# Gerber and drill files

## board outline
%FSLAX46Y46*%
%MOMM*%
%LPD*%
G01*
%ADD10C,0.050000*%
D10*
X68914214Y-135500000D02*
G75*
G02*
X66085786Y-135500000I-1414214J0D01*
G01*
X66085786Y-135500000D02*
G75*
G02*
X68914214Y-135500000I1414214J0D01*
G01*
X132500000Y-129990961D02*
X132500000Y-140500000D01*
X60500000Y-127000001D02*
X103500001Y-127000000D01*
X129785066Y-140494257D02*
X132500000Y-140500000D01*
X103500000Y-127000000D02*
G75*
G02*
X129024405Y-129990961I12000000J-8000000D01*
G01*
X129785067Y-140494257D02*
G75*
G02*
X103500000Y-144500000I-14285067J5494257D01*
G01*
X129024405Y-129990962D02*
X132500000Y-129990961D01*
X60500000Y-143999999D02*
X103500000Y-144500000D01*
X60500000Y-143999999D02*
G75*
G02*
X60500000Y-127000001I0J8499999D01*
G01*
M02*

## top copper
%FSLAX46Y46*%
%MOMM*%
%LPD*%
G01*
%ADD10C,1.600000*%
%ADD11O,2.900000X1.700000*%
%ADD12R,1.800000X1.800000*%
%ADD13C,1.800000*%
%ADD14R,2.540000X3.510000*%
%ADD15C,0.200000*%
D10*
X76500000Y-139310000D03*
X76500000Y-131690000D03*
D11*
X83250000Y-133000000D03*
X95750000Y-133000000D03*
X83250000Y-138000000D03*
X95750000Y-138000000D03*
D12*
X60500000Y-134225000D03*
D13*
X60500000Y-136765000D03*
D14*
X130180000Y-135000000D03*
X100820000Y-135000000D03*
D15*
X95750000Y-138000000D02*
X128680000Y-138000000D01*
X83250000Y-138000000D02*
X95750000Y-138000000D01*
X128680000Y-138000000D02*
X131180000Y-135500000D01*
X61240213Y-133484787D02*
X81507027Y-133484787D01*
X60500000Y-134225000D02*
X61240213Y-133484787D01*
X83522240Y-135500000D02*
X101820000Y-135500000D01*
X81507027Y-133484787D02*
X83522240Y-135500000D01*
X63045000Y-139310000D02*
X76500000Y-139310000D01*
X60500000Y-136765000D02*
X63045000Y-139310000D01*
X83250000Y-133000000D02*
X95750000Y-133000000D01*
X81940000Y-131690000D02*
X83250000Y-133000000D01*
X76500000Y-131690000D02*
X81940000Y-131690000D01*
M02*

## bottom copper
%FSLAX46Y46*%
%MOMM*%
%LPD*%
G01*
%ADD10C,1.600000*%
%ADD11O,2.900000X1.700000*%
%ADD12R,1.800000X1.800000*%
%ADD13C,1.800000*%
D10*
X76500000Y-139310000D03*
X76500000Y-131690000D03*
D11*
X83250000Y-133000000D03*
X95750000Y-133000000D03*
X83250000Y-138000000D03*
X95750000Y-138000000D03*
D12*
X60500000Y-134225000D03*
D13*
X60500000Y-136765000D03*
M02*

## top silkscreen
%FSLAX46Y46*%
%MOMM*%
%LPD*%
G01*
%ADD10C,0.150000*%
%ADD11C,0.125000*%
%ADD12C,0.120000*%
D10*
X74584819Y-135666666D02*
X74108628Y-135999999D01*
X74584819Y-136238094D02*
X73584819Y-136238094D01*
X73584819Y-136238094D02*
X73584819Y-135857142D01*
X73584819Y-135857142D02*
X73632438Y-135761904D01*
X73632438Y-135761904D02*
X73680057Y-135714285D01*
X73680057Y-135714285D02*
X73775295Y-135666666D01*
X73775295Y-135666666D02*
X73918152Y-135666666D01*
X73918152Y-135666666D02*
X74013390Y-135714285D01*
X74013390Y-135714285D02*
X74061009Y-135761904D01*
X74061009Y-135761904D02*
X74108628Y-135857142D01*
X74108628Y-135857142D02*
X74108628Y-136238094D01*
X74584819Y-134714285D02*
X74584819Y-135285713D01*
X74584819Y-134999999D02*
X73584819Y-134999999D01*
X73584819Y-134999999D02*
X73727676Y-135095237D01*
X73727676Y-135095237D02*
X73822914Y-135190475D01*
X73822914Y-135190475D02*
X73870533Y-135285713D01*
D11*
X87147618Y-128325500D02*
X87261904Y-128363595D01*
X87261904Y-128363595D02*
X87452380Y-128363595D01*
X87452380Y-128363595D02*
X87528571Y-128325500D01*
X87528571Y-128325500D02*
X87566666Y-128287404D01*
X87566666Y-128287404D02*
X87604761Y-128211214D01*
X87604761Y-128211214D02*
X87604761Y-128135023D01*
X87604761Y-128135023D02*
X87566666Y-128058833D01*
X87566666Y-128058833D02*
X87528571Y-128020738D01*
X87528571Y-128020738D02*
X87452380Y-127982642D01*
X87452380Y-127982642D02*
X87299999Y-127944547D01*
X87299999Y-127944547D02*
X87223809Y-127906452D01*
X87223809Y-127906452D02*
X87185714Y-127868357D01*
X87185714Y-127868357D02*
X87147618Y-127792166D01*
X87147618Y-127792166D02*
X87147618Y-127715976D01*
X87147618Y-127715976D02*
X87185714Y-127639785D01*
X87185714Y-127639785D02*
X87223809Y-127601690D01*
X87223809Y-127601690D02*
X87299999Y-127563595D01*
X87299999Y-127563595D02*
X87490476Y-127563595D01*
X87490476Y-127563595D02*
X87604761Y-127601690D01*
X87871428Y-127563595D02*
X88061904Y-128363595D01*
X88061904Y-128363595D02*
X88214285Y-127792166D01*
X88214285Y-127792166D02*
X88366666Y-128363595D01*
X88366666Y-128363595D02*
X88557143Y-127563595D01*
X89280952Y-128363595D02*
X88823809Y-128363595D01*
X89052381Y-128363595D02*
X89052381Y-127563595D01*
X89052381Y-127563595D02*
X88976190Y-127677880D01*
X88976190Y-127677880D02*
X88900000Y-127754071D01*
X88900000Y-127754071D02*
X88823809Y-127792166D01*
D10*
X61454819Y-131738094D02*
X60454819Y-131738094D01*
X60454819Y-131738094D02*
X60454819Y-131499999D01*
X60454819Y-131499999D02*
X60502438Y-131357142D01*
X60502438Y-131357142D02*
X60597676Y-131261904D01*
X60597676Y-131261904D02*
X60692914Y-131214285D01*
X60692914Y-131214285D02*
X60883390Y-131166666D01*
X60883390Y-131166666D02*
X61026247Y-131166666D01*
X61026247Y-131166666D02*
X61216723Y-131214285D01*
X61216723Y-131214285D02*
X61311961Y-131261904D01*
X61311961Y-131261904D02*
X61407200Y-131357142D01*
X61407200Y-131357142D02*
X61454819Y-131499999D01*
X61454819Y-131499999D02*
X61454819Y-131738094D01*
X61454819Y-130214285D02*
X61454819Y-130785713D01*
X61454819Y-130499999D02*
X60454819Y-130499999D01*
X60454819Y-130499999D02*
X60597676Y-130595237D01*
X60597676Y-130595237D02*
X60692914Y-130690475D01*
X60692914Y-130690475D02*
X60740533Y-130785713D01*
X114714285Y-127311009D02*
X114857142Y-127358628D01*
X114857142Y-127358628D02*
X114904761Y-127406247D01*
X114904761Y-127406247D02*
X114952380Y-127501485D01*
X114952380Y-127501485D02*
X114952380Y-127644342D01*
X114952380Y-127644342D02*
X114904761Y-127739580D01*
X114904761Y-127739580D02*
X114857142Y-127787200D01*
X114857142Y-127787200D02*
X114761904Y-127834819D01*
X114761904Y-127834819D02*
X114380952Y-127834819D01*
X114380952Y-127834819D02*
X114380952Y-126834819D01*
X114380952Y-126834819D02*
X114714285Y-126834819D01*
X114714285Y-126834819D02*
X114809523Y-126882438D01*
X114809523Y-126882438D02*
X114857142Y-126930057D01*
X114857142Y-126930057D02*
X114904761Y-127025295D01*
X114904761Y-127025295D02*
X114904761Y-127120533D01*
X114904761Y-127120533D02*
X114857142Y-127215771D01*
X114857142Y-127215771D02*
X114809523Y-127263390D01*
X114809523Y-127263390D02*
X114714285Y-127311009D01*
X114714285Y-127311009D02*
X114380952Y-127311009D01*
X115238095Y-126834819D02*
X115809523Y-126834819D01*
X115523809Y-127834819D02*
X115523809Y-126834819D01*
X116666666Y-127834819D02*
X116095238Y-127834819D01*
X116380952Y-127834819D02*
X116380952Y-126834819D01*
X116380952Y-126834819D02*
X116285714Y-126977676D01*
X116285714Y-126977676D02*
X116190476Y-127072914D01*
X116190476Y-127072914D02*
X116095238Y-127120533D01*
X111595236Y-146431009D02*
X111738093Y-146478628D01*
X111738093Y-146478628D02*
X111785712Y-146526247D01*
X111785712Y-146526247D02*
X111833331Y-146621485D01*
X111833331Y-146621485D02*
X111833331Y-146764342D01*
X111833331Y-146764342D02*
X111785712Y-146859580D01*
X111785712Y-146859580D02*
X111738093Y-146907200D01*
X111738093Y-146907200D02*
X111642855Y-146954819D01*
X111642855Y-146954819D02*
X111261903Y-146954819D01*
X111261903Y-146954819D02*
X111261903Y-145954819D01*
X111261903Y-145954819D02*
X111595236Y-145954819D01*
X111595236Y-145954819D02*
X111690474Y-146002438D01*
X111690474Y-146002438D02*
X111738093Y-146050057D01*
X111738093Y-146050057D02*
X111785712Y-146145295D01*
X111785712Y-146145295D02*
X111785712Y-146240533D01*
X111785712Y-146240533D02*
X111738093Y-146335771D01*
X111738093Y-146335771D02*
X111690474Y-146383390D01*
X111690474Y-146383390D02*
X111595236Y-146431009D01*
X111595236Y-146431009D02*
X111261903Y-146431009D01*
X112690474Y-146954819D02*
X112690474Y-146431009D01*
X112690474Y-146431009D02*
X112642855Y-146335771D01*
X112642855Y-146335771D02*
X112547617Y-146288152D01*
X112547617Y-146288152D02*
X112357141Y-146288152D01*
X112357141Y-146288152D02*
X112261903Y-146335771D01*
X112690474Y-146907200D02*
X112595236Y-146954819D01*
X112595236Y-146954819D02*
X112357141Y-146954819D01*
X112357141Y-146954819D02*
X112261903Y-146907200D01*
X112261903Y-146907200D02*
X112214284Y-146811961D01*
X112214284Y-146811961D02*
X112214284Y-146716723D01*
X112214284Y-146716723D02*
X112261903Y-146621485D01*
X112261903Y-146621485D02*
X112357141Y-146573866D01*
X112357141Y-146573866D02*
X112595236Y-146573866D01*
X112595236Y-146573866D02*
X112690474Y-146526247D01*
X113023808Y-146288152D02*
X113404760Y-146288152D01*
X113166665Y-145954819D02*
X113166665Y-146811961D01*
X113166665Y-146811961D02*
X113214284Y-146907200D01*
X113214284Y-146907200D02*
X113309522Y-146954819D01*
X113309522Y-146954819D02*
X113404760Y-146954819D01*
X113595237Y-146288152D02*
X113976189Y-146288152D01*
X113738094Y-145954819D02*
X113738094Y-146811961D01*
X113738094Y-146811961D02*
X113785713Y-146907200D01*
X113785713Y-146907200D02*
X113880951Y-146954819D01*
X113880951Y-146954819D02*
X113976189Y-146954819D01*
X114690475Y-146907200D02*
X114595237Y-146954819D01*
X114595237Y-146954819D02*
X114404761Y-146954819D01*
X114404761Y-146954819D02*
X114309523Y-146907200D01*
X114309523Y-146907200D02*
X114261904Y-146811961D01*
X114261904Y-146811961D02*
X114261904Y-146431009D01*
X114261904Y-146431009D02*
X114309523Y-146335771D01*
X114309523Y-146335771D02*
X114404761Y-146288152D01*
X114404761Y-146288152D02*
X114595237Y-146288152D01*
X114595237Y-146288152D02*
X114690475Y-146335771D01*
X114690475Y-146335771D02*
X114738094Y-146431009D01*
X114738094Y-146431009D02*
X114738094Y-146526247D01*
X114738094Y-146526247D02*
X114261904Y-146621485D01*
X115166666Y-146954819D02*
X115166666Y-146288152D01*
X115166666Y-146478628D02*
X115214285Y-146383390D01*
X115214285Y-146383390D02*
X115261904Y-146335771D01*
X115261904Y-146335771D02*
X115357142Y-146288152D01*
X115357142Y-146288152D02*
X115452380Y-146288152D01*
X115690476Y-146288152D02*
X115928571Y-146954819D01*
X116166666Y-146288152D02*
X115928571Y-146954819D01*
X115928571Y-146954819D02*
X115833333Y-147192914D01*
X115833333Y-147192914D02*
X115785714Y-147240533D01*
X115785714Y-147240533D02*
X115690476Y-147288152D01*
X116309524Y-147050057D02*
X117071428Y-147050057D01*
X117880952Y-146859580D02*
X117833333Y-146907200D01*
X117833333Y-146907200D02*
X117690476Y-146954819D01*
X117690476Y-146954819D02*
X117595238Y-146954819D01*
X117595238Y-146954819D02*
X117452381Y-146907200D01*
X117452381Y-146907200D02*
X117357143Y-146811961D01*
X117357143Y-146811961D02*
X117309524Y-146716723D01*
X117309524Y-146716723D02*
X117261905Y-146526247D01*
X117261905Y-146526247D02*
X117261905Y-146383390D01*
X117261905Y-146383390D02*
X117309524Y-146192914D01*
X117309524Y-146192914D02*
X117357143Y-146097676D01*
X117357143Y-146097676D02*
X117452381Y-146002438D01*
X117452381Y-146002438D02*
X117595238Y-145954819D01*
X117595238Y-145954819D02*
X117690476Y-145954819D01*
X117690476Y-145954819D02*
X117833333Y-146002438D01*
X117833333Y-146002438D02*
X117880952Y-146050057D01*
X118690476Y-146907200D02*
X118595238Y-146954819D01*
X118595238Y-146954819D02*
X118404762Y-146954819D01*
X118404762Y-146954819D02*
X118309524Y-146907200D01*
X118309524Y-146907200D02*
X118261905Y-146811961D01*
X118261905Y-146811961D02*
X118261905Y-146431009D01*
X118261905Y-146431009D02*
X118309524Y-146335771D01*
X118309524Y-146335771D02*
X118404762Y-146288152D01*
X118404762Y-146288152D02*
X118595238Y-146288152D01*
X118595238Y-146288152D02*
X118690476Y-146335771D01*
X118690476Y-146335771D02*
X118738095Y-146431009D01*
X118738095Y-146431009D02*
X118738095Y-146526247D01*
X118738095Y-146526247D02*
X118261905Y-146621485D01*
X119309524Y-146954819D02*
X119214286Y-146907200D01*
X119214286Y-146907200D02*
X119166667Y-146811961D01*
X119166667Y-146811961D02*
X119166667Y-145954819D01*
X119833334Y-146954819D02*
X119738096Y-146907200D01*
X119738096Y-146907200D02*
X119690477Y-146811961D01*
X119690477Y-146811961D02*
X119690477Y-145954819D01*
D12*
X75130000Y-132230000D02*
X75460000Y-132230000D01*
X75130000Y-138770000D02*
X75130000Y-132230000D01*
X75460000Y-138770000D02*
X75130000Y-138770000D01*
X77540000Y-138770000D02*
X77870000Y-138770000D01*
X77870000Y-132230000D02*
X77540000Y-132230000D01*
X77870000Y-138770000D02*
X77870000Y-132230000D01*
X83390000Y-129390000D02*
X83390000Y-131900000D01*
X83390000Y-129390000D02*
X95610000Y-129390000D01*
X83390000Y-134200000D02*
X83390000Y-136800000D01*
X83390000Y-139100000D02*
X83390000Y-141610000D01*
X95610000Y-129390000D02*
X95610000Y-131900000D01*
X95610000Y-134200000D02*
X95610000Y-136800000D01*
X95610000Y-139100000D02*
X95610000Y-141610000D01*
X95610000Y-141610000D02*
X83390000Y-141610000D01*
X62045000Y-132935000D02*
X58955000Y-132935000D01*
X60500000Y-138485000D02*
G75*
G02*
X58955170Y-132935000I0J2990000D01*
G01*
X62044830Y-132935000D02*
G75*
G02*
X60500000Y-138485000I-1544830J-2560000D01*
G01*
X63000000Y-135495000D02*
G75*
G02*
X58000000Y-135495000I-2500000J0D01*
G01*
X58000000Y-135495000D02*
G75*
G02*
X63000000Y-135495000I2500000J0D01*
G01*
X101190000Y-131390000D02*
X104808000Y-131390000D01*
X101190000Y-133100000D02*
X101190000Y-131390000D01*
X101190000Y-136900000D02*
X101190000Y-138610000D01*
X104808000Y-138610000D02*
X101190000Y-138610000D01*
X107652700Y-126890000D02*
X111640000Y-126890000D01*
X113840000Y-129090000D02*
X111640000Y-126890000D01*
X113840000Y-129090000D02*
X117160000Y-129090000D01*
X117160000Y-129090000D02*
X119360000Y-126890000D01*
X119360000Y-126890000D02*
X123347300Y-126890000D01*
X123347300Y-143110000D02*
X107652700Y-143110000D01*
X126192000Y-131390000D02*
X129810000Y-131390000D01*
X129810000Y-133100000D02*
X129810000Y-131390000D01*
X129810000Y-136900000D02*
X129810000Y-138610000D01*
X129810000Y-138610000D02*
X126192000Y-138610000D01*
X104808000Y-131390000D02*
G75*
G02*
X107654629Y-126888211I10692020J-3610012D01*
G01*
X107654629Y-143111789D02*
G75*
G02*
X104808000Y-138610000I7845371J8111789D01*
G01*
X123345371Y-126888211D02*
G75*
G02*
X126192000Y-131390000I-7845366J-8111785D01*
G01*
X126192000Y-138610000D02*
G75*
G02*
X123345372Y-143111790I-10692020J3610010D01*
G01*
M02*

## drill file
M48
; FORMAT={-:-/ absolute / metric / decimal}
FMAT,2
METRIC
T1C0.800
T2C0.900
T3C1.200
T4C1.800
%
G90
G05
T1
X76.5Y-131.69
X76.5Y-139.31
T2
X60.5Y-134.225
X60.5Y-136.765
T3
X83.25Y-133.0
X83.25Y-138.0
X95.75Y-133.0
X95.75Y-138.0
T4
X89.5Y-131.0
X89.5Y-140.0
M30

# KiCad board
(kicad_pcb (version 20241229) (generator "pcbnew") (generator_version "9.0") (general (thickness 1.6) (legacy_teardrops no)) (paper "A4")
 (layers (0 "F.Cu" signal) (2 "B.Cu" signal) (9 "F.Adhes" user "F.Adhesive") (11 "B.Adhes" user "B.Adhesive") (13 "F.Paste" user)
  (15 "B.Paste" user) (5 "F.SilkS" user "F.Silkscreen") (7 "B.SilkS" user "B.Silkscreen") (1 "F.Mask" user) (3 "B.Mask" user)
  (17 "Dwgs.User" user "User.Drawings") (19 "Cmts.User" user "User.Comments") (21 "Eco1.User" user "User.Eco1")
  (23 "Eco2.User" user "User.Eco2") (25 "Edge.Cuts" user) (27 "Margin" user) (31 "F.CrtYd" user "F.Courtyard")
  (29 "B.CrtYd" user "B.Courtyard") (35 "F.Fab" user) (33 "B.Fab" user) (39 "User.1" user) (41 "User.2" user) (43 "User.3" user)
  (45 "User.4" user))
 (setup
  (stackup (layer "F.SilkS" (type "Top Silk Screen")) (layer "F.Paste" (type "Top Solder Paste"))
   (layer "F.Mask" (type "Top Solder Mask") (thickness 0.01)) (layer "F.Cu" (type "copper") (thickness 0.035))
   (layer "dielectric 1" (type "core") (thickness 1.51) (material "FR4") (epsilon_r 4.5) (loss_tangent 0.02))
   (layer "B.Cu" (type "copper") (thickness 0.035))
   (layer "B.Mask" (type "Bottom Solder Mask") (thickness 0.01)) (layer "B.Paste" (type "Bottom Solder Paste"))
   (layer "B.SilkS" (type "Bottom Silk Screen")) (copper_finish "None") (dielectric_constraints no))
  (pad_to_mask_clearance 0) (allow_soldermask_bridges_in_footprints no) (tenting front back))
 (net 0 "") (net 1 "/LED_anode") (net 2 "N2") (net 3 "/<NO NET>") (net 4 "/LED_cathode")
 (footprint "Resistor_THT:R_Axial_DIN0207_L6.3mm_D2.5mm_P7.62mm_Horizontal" (layer "F.Cu") (at 76.5 139.31 90)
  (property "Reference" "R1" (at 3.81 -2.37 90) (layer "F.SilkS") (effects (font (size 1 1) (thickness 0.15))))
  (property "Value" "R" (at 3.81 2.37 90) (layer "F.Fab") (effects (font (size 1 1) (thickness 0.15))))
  (fp_line (start 7.08 -1.37) (end 7.08 -1.04) (stroke (width 0.12) (type solid)) (layer "F.SilkS"))
  (fp_line (start 0.54 -1.37) (end 7.08 -1.37) (stroke (width 0.12) (type solid)) (layer "F.SilkS"))
  (fp_line (start 0.54 -1.04) (end 0.54 -1.37) (stroke (width 0.12) (type solid)) (layer "F.SilkS"))
  (fp_line (start 0.54 1.04) (end 0.54 1.37) (stroke (width 0.12) (type solid)) (layer "F.SilkS"))
  (fp_line (start 7.08 1.37) (end 7.08 1.04) (stroke (width 0.12) (type solid)) (layer "F.SilkS"))
  (fp_line (start 0.54 1.37) (end 7.08 1.37) (stroke (width 0.12) (type solid)) (layer "F.SilkS"))
  (pad "1" thru_hole circle (at 0 0 90) (size 1.6 1.6) (drill 0.8) (layers "*.Cu" "*.Mask") (remove_unused_layers no) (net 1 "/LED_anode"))
  (pad "2" thru_hole circle (at 7.62 0 90) (size 1.6 1.6) (drill 0.8) (layers "*.Cu" "*.Mask") (remove_unused_layers no) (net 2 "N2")))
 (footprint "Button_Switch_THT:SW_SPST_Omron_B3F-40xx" (layer "F.Cu") (at 83.25 133)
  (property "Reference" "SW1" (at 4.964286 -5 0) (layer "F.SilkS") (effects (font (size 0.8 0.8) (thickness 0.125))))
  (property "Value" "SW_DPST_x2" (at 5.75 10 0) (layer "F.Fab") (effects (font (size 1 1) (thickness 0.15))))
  (fp_line (start 0.14 -3.61) (end 0.14 -1.1) (stroke (width 0.12) (type default)) (layer "F.SilkS"))
  (fp_line (start 0.14 -3.61) (end 12.36 -3.61) (stroke (width 0.12) (type default)) (layer "F.SilkS"))
  (fp_line (start 0.14 1.2) (end 0.14 3.8) (stroke (width 0.12) (type default)) (layer "F.SilkS"))
  (fp_line (start 0.14 6.1) (end 0.14 8.61) (stroke (width 0.12) (type default)) (layer "F.SilkS"))
  (fp_line (start 12.36 -3.61) (end 12.36 -1.1) (stroke (width 0.12) (type default)) (layer "F.SilkS"))
  (fp_line (start 12.36 1.2) (end 12.36 3.8) (stroke (width 0.12) (type default)) (layer "F.SilkS"))
  (fp_line (start 12.36 6.1) (end 12.36 8.61) (stroke (width 0.12) (type default)) (layer "F.SilkS"))
  (fp_line (start 12.36 8.61) (end 0.14 8.61) (stroke (width 0.12) (type default)) (layer "F.SilkS"))
  (pad "" np_thru_hole circle (at 6.25 -2) (size 1.8 1.8) (drill 1.8) (layers "*.Cu" "*.Mask"))
  (pad "" np_thru_hole circle (at 6.25 7) (size 1.8 1.8) (drill 1.8) (layers "*.Cu" "*.Mask"))
  (pad "1" thru_hole oval (at 0 0) (size 2.9 1.7) (drill 1.2) (layers "*.Cu" "*.Mask") (remove_unused_layers no) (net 2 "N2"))
  (pad "1" thru_hole oval (at 12.5 0) (size 2.9 1.7) (drill 1.2) (layers "*.Cu" "*.Mask") (remove_unused_layers no) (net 2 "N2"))
  (pad "2" thru_hole oval (at 0 5) (size 2.9 1.7) (drill 1.2) (layers "*.Cu" "*.Mask") (remove_unused_layers no) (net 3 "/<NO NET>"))
  (pad "2" thru_hole oval (at 12.5 5) (size 2.9 1.7) (drill 1.2) (layers "*.Cu" "*.Mask") (remove_unused_layers no) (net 3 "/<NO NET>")))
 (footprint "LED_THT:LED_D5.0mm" (layer "F.Cu") (at 60.5 134.225 -90)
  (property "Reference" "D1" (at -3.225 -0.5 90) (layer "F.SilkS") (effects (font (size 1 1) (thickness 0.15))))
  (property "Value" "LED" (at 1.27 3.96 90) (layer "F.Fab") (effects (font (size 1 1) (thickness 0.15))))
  (fp_line (start -1.29 -1.545) (end -1.29 1.545) (stroke (width 0.12) (type solid)) (layer "F.SilkS"))
  (fp_arc (start 4.26 0) (mid 2.071779 2.880495) (end -1.29 1.54483) (stroke (width 0.12) (type solid)) (layer "F.SilkS"))
  (fp_arc (start -1.29 -1.54483) (mid 2.071779 -2.880495) (end 4.26 0) (stroke (width 0.12) (type solid)) (layer "F.SilkS"))
  (fp_circle (center 1.27 0) (end 3.77 0) (stroke (width 0.12) (type solid)) (fill no) (layer "F.SilkS"))
  (pad "1" thru_hole rect (at 0 0 270) (size 1.8 1.8) (drill 0.9) (layers "*.Cu" "*.Mask") (remove_unused_layers no) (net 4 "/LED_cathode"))
  (pad "2" thru_hole circle (at 2.54 0 270) (size 1.8 1.8) (drill 0.9) (layers "*.Cu" "*.Mask") (remove_unused_layers no)
   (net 1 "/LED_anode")))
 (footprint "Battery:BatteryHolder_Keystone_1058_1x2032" (layer "F.Cu") (at 115.5 135 180)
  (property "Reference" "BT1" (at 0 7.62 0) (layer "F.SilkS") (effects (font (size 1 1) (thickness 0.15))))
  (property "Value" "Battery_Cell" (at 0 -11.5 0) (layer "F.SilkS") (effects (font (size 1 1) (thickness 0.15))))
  (fp_line (start 14.31 3.61) (end 10.692 3.61) (stroke (width 0.12) (type solid)) (layer "F.SilkS"))
  (fp_line (start 14.31 1.9) (end 14.31 3.61) (stroke (width 0.12) (type solid)) (layer "F.SilkS"))
  (fp_line (start 14.31 -1.9) (end 14.31 -3.61) (stroke (width 0.12) (type solid)) (layer "F.SilkS"))
  (fp_line (start 10.692 -3.61) (end 14.31 -3.61) (stroke (width 0.12) (type solid)) (layer "F.SilkS"))
  (fp_line (start 7.8473 8.11) (end 3.86 8.11) (stroke (width 0.12) (type solid)) (layer "F.SilkS"))
  (fp_line (start 1.66 5.91) (end 3.86 8.11) (stroke (width 0.12) (type solid)) (layer "F.SilkS"))
  (fp_line (start 1.66 5.91) (end -1.66 5.91) (stroke (width 0.12) (type solid)) (layer "F.SilkS"))
  (fp_line (start -1.66 5.91) (end -3.86 8.11) (stroke (width 0.12) (type solid)) (layer "F.SilkS"))
  (fp_line (start -3.86 8.11) (end -7.8473 8.11) (stroke (width 0.12) (type solid)) (layer "F.SilkS"))
  (fp_line (start -7.8473 -8.11) (end 7.8473 -8.11) (stroke (width 0.12) (type solid)) (layer "F.SilkS"))
  (fp_line (start -10.692 3.61) (end -14.31 3.61) (stroke (width 0.12) (type solid)) (layer "F.SilkS"))
  (fp_line (start -14.31 1.9) (end -14.31 3.61) (stroke (width 0.12) (type solid)) (layer "F.SilkS"))
  (fp_line (start -14.31 -1.9) (end -14.31 -3.61) (stroke (width 0.12) (type solid)) (layer "F.SilkS"))
  (fp_line (start -14.31 -3.61) (end -10.692 -3.61) (stroke (width 0.12) (type solid)) (layer "F.SilkS"))
  (fp_arc (start 10.692 3.61) (mid 9.538084 6.031244) (end 7.845371 8.111789) (stroke (width 0.12) (type solid)) (layer "F.SilkS"))
  (fp_arc (start 7.845371 -8.111789) (mid 9.538085 -6.031244) (end 10.692 -3.61) (stroke (width 0.12) (type solid)) (layer "F.SilkS"))
  (fp_arc (start -7.845371 8.111789) (mid -9.538085 6.031244) (end -10.692 3.61) (stroke (width 0.12) (type solid)) (layer "F.SilkS"))
  (fp_arc (start -10.692 -3.61) (mid -9.538084 -6.031244) (end -7.845371 -8.111789) (stroke (width 0.12) (type solid)) (layer "F.SilkS"))
  (pad "1" smd rect (at -14.68 0 180) (size 2.54 3.51) (layers "F.Cu" "F.Mask" "F.Paste") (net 3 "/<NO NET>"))
  (pad "2" smd rect (at 14.68 0 180) (size 2.54 3.51) (layers "F.Cu" "F.Mask" "F.Paste") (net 4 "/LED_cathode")))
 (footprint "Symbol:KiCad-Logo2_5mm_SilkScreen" (layer "B.Cu") (at 115.5 133 180)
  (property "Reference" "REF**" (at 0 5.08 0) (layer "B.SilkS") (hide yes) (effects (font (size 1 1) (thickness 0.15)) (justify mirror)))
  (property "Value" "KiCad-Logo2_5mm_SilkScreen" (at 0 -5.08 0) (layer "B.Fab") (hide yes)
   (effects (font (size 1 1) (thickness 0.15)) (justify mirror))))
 (gr_circle (center 67.5 135.5) (end 68.5 136.5) (stroke (width 0.05) (type default)) (fill no) (locked yes) (layer "Edge.Cuts"))
 (gr_line (start 132.5 129.990961) (end 132.5 140.5) (stroke (width 0.05) (type default)) (locked yes) (layer "Edge.Cuts"))
 (gr_line (start 60.5 127.000001) (end 103.500001 127) (stroke (width 0.05) (type default)) (locked yes) (layer "Edge.Cuts"))
 (gr_line (start 129.785066 140.494257) (end 132.5 140.5) (stroke (width 0.05) (type default)) (locked yes) (layer "Edge.Cuts"))
 (gr_arc (start 103.5 127) (mid 117.178516 120.675804) (end 129.024405 129.990961) (stroke (width 0.05) (type default)) (locked yes)
  (layer "Edge.Cuts"))
 (gr_arc (start 129.785067 140.494257) (mid 117.805835 150.130536) (end 103.5 144.5) (stroke (width 0.05) (type default)) (locked yes)
  (layer "Edge.Cuts"))
 (gr_line (start 129.024405 129.990962) (end 132.5 129.990961) (stroke (width 0.05) (type default)) (locked yes) (layer "Edge.Cuts"))
 (gr_line (start 60.5 143.999999) (end 103.5 144.5) (stroke (width 0.05) (type default)) (locked yes) (layer "Edge.Cuts"))
 (gr_arc (start 60.5 143.999999) (mid 52.000001 135.5) (end 60.5 127.000001) (stroke (width 0.05) (type default)) (locked yes)
  (layer "Edge.Cuts"))
 (segment (start 95.75 138) (end 128.68 138) (width 0.2) (layer "F.Cu") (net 3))
 (segment (start 83.25 138) (end 95.75 138) (width 0.2) (layer "F.Cu") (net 3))
 (segment (start 128.68 138) (end 131.18 135.5) (width 0.2) (layer "F.Cu") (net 3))
 (segment (start 61.240213 133.484787) (end 81.507027 133.484787) (width 0.2) (layer "F.Cu") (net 4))
 (segment (start 60.5 134.225) (end 61.240213 133.484787) (width 0.2) (layer "F.Cu") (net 4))
 (segment (start 83.52224 135.5) (end 101.82 135.5) (width 0.2) (layer "F.Cu") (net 4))
 (segment (start 81.507027 133.484787) (end 83.52224 135.5) (width 0.2) (layer "F.Cu") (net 4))
 (segment (start 63.045 139.31) (end 76.5 139.31) (width 0.2) (layer "F.Cu") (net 1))
 (segment (start 60.5 136.765) (end 63.045 139.31) (width 0.2) (layer "F.Cu") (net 1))
 (segment (start 83.25 133) (end 95.75 133) (width 0.2) (layer "F.Cu") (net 2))
 (segment (start 81.94 131.69) (end 83.25 133) (width 0.2) (layer "F.Cu") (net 2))
 (segment (start 76.5 131.69) (end 81.94 131.69) (width 0.2) (layer "F.Cu") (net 2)))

